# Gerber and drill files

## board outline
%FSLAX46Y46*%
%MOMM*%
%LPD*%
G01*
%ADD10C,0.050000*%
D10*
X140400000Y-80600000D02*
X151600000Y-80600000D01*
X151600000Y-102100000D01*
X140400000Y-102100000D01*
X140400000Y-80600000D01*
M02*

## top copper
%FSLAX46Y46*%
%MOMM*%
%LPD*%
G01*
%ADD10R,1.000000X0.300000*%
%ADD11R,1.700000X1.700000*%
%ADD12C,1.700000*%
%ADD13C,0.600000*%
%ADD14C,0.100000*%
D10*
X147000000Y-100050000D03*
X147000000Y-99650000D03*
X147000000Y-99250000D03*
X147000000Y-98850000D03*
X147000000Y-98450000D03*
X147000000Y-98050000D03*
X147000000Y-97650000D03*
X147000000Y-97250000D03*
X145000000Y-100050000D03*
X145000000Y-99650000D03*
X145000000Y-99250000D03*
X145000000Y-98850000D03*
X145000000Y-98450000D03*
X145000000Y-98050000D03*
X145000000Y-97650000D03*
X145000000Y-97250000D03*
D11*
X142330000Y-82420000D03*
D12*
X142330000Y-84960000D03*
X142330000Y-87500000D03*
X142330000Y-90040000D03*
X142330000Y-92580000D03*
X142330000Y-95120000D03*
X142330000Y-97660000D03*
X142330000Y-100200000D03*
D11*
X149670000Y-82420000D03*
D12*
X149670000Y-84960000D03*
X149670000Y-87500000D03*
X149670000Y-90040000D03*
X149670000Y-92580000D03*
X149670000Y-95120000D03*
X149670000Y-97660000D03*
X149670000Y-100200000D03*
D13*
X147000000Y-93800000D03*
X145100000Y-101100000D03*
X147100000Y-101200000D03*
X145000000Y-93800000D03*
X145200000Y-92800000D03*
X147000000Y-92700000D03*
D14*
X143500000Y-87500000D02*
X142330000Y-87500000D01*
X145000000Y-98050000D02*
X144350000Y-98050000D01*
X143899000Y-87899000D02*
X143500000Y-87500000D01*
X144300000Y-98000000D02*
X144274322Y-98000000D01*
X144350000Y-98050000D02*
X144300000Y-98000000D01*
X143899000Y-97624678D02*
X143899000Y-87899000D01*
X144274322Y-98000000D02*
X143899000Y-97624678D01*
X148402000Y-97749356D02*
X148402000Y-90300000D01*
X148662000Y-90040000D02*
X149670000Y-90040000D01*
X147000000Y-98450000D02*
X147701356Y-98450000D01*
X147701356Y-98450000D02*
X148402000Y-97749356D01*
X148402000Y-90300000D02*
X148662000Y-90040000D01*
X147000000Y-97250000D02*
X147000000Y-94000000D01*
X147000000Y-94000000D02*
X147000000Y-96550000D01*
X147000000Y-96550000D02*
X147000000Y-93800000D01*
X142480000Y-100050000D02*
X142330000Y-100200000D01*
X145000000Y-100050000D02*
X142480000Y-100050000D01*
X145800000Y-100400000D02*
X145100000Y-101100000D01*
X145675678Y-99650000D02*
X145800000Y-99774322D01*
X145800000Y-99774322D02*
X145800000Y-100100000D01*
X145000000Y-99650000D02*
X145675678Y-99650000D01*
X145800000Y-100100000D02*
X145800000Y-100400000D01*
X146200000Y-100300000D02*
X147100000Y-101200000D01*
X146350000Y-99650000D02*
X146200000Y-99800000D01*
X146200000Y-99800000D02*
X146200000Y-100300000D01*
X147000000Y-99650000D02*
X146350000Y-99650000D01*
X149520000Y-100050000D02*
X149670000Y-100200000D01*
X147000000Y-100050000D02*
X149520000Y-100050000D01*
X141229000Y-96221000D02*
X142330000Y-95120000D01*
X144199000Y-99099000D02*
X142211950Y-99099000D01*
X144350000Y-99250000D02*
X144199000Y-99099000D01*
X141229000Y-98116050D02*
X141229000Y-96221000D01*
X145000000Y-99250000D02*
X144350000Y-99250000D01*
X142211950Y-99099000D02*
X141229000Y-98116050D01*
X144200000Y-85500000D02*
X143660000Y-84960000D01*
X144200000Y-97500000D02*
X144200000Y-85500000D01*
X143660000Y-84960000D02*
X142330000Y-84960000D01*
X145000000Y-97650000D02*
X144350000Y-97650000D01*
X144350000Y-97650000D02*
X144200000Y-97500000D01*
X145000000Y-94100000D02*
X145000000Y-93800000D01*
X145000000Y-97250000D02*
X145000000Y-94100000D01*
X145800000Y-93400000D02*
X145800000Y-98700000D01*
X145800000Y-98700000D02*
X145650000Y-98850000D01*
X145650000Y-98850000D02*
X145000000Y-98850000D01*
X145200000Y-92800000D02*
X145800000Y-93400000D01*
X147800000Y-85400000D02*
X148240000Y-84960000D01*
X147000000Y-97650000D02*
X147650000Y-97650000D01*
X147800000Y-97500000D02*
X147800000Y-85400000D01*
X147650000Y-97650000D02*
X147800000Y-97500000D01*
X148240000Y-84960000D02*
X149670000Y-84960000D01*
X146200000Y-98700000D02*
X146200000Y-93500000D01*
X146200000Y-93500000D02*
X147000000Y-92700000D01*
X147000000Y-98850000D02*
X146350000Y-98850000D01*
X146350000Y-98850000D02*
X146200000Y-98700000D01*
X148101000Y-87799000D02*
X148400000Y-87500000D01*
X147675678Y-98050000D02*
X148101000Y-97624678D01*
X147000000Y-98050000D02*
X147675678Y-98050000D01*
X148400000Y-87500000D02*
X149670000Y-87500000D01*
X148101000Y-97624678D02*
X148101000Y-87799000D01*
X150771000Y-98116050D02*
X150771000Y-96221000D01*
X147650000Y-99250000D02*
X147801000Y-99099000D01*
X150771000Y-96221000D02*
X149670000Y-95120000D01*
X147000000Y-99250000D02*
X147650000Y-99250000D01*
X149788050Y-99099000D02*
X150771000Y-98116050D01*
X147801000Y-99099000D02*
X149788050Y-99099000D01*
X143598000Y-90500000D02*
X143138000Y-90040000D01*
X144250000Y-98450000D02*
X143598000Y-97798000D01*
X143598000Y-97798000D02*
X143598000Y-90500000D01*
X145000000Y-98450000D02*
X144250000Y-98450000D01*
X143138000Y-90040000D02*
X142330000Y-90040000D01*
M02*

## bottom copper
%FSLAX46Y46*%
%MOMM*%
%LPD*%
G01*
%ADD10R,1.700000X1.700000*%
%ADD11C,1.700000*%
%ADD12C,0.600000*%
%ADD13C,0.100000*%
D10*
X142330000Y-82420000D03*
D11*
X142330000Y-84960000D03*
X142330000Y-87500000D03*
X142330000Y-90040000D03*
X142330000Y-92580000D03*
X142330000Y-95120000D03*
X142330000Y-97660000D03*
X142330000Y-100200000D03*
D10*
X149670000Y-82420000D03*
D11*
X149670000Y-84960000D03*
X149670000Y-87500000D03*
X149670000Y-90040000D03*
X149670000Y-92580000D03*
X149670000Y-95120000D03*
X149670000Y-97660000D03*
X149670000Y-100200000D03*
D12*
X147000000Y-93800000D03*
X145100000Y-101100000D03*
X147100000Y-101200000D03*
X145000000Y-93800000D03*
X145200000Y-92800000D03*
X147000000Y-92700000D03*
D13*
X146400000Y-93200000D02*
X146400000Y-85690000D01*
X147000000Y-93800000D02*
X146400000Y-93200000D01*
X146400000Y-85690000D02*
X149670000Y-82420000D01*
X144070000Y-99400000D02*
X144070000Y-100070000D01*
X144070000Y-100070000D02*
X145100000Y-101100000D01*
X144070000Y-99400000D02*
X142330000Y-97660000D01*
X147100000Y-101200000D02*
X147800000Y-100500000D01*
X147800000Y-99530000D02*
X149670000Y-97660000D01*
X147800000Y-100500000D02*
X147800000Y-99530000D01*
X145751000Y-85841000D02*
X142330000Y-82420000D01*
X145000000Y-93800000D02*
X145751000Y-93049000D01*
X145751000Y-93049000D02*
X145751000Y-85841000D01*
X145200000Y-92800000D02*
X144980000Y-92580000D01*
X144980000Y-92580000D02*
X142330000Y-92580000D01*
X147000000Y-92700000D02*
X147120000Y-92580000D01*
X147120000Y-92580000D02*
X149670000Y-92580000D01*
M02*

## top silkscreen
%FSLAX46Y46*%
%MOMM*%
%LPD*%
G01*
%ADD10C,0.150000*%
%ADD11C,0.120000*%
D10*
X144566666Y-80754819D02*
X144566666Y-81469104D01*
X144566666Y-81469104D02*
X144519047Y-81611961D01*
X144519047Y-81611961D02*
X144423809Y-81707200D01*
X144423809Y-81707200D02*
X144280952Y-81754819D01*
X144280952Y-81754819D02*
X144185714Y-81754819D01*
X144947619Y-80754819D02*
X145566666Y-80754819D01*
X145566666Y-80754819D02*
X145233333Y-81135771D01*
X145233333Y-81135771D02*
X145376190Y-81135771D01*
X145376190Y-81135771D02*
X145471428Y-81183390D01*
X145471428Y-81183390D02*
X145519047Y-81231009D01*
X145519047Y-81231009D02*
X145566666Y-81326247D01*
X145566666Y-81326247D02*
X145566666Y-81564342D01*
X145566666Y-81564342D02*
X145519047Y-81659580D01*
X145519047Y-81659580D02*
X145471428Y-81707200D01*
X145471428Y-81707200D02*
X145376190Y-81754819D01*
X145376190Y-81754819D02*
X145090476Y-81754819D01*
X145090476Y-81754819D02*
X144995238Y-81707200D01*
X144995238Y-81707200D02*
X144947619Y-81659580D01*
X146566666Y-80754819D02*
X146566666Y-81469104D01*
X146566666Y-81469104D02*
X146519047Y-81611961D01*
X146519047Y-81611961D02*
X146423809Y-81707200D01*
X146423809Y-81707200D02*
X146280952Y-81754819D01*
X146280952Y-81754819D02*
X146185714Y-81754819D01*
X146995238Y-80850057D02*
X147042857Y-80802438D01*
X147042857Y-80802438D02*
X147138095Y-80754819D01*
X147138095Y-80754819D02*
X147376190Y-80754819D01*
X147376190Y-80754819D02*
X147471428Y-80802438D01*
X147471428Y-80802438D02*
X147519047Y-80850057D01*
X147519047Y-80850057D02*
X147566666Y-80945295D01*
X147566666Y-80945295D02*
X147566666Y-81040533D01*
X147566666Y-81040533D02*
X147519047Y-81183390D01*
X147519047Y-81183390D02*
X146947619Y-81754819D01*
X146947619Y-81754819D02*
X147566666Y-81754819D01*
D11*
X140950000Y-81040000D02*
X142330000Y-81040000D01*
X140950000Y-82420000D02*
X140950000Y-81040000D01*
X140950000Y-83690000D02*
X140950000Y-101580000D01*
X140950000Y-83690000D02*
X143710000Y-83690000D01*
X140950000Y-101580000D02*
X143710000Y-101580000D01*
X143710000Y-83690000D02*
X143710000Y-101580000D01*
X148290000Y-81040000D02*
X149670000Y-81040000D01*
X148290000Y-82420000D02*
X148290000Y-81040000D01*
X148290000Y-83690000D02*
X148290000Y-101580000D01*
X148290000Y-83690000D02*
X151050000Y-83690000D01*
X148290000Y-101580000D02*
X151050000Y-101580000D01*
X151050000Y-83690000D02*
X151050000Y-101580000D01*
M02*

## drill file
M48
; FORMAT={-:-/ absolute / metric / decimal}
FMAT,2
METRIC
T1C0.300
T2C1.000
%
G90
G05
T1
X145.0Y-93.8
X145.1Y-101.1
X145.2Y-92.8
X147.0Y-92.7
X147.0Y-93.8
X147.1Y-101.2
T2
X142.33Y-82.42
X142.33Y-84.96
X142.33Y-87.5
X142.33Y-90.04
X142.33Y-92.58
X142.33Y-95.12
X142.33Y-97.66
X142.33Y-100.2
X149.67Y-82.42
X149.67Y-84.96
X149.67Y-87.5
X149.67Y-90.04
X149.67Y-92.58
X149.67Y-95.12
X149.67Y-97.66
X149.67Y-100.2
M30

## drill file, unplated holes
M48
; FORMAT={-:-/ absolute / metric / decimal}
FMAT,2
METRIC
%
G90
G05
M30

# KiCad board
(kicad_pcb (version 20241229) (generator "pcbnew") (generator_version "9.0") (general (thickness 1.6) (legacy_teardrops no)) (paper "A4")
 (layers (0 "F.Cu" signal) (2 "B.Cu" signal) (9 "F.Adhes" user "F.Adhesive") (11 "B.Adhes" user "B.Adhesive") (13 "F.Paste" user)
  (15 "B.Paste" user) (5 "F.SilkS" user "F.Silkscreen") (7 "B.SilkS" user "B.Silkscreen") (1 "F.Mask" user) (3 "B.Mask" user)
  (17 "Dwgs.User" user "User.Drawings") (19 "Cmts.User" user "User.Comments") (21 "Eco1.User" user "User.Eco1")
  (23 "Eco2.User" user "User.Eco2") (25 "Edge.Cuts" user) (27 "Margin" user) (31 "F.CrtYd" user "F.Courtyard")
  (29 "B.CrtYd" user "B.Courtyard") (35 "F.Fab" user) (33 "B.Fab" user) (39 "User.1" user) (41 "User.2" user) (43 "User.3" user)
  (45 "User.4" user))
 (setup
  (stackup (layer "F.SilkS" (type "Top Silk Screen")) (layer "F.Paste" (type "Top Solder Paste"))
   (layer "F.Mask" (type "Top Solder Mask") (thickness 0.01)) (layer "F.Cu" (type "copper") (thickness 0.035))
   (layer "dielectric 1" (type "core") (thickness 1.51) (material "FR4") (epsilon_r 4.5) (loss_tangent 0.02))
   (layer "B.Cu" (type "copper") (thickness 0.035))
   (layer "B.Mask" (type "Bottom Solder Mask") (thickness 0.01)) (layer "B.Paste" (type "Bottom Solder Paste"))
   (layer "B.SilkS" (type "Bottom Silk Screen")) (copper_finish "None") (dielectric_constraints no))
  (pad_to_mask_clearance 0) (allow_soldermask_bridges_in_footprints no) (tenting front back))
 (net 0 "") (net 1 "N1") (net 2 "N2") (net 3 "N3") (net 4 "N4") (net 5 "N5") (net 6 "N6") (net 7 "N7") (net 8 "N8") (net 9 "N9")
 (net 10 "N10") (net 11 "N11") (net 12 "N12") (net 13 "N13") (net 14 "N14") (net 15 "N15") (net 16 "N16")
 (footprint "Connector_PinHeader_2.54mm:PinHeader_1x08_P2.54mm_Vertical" (layer "F.Cu") (at 142.33 82.42)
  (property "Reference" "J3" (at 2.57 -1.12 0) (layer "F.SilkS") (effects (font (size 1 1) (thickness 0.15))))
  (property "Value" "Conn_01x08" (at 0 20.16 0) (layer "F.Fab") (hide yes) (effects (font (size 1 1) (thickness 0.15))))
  (fp_line (start -1.38 -1.38) (end 0 -1.38) (stroke (width 0.12) (type solid)) (layer "F.SilkS"))
  (fp_line (start -1.38 0) (end -1.38 -1.38) (stroke (width 0.12) (type solid)) (layer "F.SilkS"))
  (fp_line (start -1.38 1.27) (end -1.38 19.16) (stroke (width 0.12) (type solid)) (layer "F.SilkS"))
  (fp_line (start -1.38 1.27) (end 1.38 1.27) (stroke (width 0.12) (type solid)) (layer "F.SilkS"))
  (fp_line (start -1.38 19.16) (end 1.38 19.16) (stroke (width 0.12) (type solid)) (layer "F.SilkS"))
  (fp_line (start 1.38 1.27) (end 1.38 19.16) (stroke (width 0.12) (type solid)) (layer "F.SilkS"))
  (pad "1" thru_hole rect (at 0 0) (size 1.7 1.7) (drill 1) (layers "*.Cu" "*.Mask") (remove_unused_layers no) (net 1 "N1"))
  (pad "2" thru_hole circle (at 0 2.54) (size 1.7 1.7) (drill 1) (layers "*.Cu" "*.Mask") (remove_unused_layers no) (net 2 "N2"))
  (pad "3" thru_hole circle (at 0 5.08) (size 1.7 1.7) (drill 1) (layers "*.Cu" "*.Mask") (remove_unused_layers no) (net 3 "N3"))
  (pad "4" thru_hole circle (at 0 7.62) (size 1.7 1.7) (drill 1) (layers "*.Cu" "*.Mask") (remove_unused_layers no) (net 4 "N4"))
  (pad "5" thru_hole circle (at 0 10.16) (size 1.7 1.7) (drill 1) (layers "*.Cu" "*.Mask") (remove_unused_layers no) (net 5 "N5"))
  (pad "6" thru_hole circle (at 0 12.7) (size 1.7 1.7) (drill 1) (layers "*.Cu" "*.Mask") (remove_unused_layers no) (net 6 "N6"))
  (pad "7" thru_hole circle (at 0 15.24) (size 1.7 1.7) (drill 1) (layers "*.Cu" "*.Mask") (remove_unused_layers no) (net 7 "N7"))
  (pad "8" thru_hole circle (at 0 17.78) (size 1.7 1.7) (drill 1) (layers "*.Cu" "*.Mask") (remove_unused_layers no) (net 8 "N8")))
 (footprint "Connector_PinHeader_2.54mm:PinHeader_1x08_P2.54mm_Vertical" (layer "F.Cu") (at 149.67 82.42)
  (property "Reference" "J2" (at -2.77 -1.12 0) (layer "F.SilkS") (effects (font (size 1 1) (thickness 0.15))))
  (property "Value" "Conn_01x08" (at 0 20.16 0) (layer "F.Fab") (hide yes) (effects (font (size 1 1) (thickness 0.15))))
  (fp_line (start -1.38 -1.38) (end 0 -1.38) (stroke (width 0.12) (type solid)) (layer "F.SilkS"))
  (fp_line (start -1.38 0) (end -1.38 -1.38) (stroke (width 0.12) (type solid)) (layer "F.SilkS"))
  (fp_line (start -1.38 1.27) (end -1.38 19.16) (stroke (width 0.12) (type solid)) (layer "F.SilkS"))
  (fp_line (start -1.38 1.27) (end 1.38 1.27) (stroke (width 0.12) (type solid)) (layer "F.SilkS"))
  (fp_line (start -1.38 19.16) (end 1.38 19.16) (stroke (width 0.12) (type solid)) (layer "F.SilkS"))
  (fp_line (start 1.38 1.27) (end 1.38 19.16) (stroke (width 0.12) (type solid)) (layer "F.SilkS"))
  (pad "1" thru_hole rect (at 0 0) (size 1.7 1.7) (drill 1) (layers "*.Cu" "*.Mask") (remove_unused_layers no) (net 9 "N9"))
  (pad "2" thru_hole circle (at 0 2.54) (size 1.7 1.7) (drill 1) (layers "*.Cu" "*.Mask") (remove_unused_layers no) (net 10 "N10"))
  (pad "3" thru_hole circle (at 0 5.08) (size 1.7 1.7) (drill 1) (layers "*.Cu" "*.Mask") (remove_unused_layers no) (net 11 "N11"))
  (pad "4" thru_hole circle (at 0 7.62) (size 1.7 1.7) (drill 1) (layers "*.Cu" "*.Mask") (remove_unused_layers no) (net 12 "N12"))
  (pad "5" thru_hole circle (at 0 10.16) (size 1.7 1.7) (drill 1) (layers "*.Cu" "*.Mask") (remove_unused_layers no) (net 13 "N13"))
  (pad "6" thru_hole circle (at 0 12.7) (size 1.7 1.7) (drill 1) (layers "*.Cu" "*.Mask") (remove_unused_layers no) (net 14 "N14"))
  (pad "7" thru_hole circle (at 0 15.24) (size 1.7 1.7) (drill 1) (layers "*.Cu" "*.Mask") (remove_unused_layers no) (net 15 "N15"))
  (pad "8" thru_hole circle (at 0 17.78) (size 1.7 1.7) (drill 1) (layers "*.Cu" "*.Mask") (remove_unused_layers no) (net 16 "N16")))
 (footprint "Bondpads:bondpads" (layer "F.Cu") (at 146 100.65)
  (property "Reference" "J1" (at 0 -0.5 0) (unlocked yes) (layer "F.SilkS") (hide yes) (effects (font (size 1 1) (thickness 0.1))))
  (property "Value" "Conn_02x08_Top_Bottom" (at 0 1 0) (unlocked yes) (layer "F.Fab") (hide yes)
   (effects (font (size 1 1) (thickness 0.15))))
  (pad "1" smd rect (at -1 -3.4) (size 1 0.3) (layers "F.Cu" "F.Mask" "F.Paste") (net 1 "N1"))
  (pad "2" smd rect (at -1 -3) (size 1 0.3) (layers "F.Cu" "F.Mask" "F.Paste") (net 2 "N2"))
  (pad "3" smd rect (at -1 -2.6) (size 1 0.3) (layers "F.Cu" "F.Mask" "F.Paste") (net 3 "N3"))
  (pad "4" smd rect (at -1 -2.2) (size 1 0.3) (layers "F.Cu" "F.Mask" "F.Paste") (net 4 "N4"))
  (pad "5" smd rect (at -1 -1.8) (size 1 0.3) (layers "F.Cu" "F.Mask" "F.Paste") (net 5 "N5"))
  (pad "6" smd rect (at -1 -1.4) (size 1 0.3) (layers "F.Cu" "F.Mask" "F.Paste") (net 6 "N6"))
  (pad "7" smd rect (at -1 -1) (size 1 0.3) (layers "F.Cu" "F.Mask" "F.Paste") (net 7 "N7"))
  (pad "8" smd rect (at -1 -0.6) (size 1 0.3) (layers "F.Cu" "F.Mask" "F.Paste") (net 8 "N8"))
  (pad "9" smd rect (at 1 -3.4) (size 1 0.3) (layers "F.Cu" "F.Mask" "F.Paste") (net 9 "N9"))
  (pad "10" smd rect (at 1 -3) (size 1 0.3) (layers "F.Cu" "F.Mask" "F.Paste") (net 10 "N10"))
  (pad "11" smd rect (at 1 -2.6) (size 1 0.3) (layers "F.Cu" "F.Mask" "F.Paste") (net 11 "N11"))
  (pad "12" smd rect (at 1 -2.2) (size 1 0.3) (layers "F.Cu" "F.Mask" "F.Paste") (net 12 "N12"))
  (pad "13" smd rect (at 1 -1.8) (size 1 0.3) (layers "F.Cu" "F.Mask" "F.Paste") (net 13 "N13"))
  (pad "14" smd rect (at 1 -1.4) (size 1 0.3) (layers "F.Cu" "F.Mask" "F.Paste") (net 14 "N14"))
  (pad "15" smd rect (at 1 -1) (size 1 0.3) (layers "F.Cu" "F.Mask" "F.Paste") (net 15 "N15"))
  (pad "16" smd rect (at 1 -0.6) (size 1 0.3) (layers "F.Cu" "F.Mask" "F.Paste") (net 16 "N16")))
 (gr_rect (start 140.4 80.6) (end 151.6 102.1) (stroke (width 0.05) (type default)) (fill no) (layer "Edge.Cuts"))
 (segment (start 143.5 87.5) (end 142.33 87.5) (width 0.1) (layer "F.Cu") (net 3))
 (segment (start 145 98.05) (end 144.35 98.05) (width 0.1) (layer "F.Cu") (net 3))
 (segment (start 143.899 87.899) (end 143.5 87.5) (width 0.1) (layer "F.Cu") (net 3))
 (segment (start 144.3 98) (end 144.274322 98) (width 0.1) (layer "F.Cu") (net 3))
 (segment (start 144.35 98.05) (end 144.3 98) (width 0.1) (layer "F.Cu") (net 3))
 (segment (start 143.899 97.624678) (end 143.899 87.899) (width 0.1) (layer "F.Cu") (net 3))
 (segment (start 144.274322 98) (end 143.899 97.624678) (width 0.1) (layer "F.Cu") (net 3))
 (segment (start 148.402 97.749356) (end 148.402 90.3) (width 0.1) (layer "F.Cu") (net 12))
 (segment (start 148.662 90.04) (end 149.67 90.04) (width 0.1) (layer "F.Cu") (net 12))
 (segment (start 147 98.45) (end 147.701356 98.45) (width 0.1) (layer "F.Cu") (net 12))
 (segment (start 147.701356 98.45) (end 148.402 97.749356) (width 0.1) (layer "F.Cu") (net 12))
 (segment (start 148.402 90.3) (end 148.662 90.04) (width 0.1) (layer "F.Cu") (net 12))
 (segment (start 147 97.25) (end 147 94) (width 0.1) (layer "F.Cu") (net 9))
 (segment (start 147 94) (end 147 96.55) (width 0.1) (layer "F.Cu") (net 9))
 (segment (start 147 96.55) (end 147 93.8) (width 0.1) (layer "F.Cu") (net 9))
 (via (at 147 93.8) (size 0.6) (drill 0.3) (layers "F.Cu" "B.Cu") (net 9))
 (segment (start 146.4 93.2) (end 146.4 85.69) (width 0.1) (layer "B.Cu") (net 9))
 (segment (start 147 93.8) (end 146.4 93.2) (width 0.1) (layer "B.Cu") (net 9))
 (segment (start 146.4 85.69) (end 149.67 82.42) (width 0.1) (layer "B.Cu") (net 9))
 (segment (start 142.48 100.05) (end 142.33 100.2) (width 0.1) (layer "F.Cu") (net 8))
 (segment (start 145 100.05) (end 142.48 100.05) (width 0.1) (layer "F.Cu") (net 8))
 (segment (start 145.8 100.4) (end 145.1 101.1) (width 0.1) (layer "F.Cu") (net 7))
 (segment (start 145.675678 99.65) (end 145.8 99.774322) (width 0.1) (layer "F.Cu") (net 7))
 (segment (start 145.8 99.774322) (end 145.8 100.1) (width 0.1) (layer "F.Cu") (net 7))
 (segment (start 145 99.65) (end 145.675678 99.65) (width 0.1) (layer "F.Cu") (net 7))
 (segment (start 145.8 100.1) (end 145.8 100.4) (width 0.1) (layer "F.Cu") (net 7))
 (via (at 145.1 101.1) (size 0.6) (drill 0.3) (layers "F.Cu" "B.Cu") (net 7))
 (segment (start 144.07 99.4) (end 144.07 100.07) (width 0.1) (layer "B.Cu") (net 7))
 (segment (start 144.07 100.07) (end 145.1 101.1) (width 0.1) (layer "B.Cu") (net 7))
 (segment (start 144.07 99.4) (end 142.33 97.66) (width 0.1) (layer "B.Cu") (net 7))
 (segment (start 146.2 100.3) (end 147.1 101.2) (width 0.1) (layer "F.Cu") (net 15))
 (segment (start 146.35 99.65) (end 146.2 99.8) (width 0.1) (layer "F.Cu") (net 15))
 (segment (start 146.2 99.8) (end 146.2 100.3) (width 0.1) (layer "F.Cu") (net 15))
 (segment (start 147 99.65) (end 146.35 99.65) (width 0.1) (layer "F.Cu") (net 15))
 (via (at 147.1 101.2) (size 0.6) (drill 0.3) (layers "F.Cu" "B.Cu") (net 15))
 (segment (start 147.1 101.2) (end 147.8 100.5) (width 0.1) (layer "B.Cu") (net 15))
 (segment (start 147.8 99.53) (end 149.67 97.66) (width 0.1) (layer "B.Cu") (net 15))
 (segment (start 147.8 100.5) (end 147.8 99.53) (width 0.1) (layer "B.Cu") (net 15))
 (segment (start 149.52 100.05) (end 149.67 100.2) (width 0.1) (layer "F.Cu") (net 16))
 (segment (start 147 100.05) (end 149.52 100.05) (width 0.1) (layer "F.Cu") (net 16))
 (segment (start 141.229 96.221) (end 142.33 95.12) (width 0.1) (layer "F.Cu") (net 6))
 (segment (start 144.199 99.099) (end 142.21195 99.099) (width 0.1) (layer "F.Cu") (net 6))
 (segment (start 144.35 99.25) (end 144.199 99.099) (width 0.1) (layer "F.Cu") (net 6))
 (segment (start 141.229 98.11605) (end 141.229 96.221) (width 0.1) (layer "F.Cu") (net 6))
 (segment (start 145 99.25) (end 144.35 99.25) (width 0.1) (layer "F.Cu") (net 6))
 (segment (start 142.21195 99.099) (end 141.229 98.11605) (width 0.1) (layer "F.Cu") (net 6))
 (segment (start 144.2 85.5) (end 143.66 84.96) (width 0.1) (layer "F.Cu") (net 2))
 (segment (start 144.2 97.5) (end 144.2 85.5) (width 0.1) (layer "F.Cu") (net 2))
 (segment (start 143.66 84.96) (end 142.33 84.96) (width 0.1) (layer "F.Cu") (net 2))
 (segment (start 145 97.65) (end 144.35 97.65) (width 0.1) (layer "F.Cu") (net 2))
 (segment (start 144.35 97.65) (end 144.2 97.5) (width 0.1) (layer "F.Cu") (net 2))
 (segment (start 145 94.1) (end 145 93.8) (width 0.1) (layer "F.Cu") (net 1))
 (segment (start 145 97.25) (end 145 94.1) (width 0.1) (layer "F.Cu") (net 1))
 (via (at 145 93.8) (size 0.6) (drill 0.3) (layers "F.Cu" "B.Cu") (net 1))
 (segment (start 145.751 85.841) (end 142.33 82.42) (width 0.1) (layer "B.Cu") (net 1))
 (segment (start 145 93.8) (end 145.751 93.049) (width 0.1) (layer "B.Cu") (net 1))
 (segment (start 145.751 93.049) (end 145.751 85.841) (width 0.1) (layer "B.Cu") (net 1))
 (segment (start 145.8 93.4) (end 145.8 98.7) (width 0.1) (layer "F.Cu") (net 5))
 (segment (start 145.8 98.7) (end 145.65 98.85) (width 0.1) (layer "F.Cu") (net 5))
 (segment (start 145.65 98.85) (end 145 98.85) (width 0.1) (layer "F.Cu") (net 5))
 (segment (start 145.2 92.8) (end 145.8 93.4) (width 0.1) (layer "F.Cu") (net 5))
 (via (at 145.2 92.8) (size 0.6) (drill 0.3) (layers "F.Cu" "B.Cu") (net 5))
 (segment (start 145.2 92.8) (end 144.98 92.58) (width 0.1) (layer "B.Cu") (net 5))
 (segment (start 144.98 92.58) (end 142.33 92.58) (width 0.1) (layer "B.Cu") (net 5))
 (segment (start 147.8 85.4) (end 148.24 84.96) (width 0.1) (layer "F.Cu") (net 10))
 (segment (start 147 97.65) (end 147.65 97.65) (width 0.1) (layer "F.Cu") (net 10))
 (segment (start 147.8 97.5) (end 147.8 85.4) (width 0.1) (layer "F.Cu") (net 10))
 (segment (start 147.65 97.65) (end 147.8 97.5) (width 0.1) (layer "F.Cu") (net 10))
 (segment (start 148.24 84.96) (end 149.67 84.96) (width 0.1) (layer "F.Cu") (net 10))
 (segment (start 146.2 98.7) (end 146.2 93.5) (width 0.1) (layer "F.Cu") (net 13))
 (segment (start 146.2 93.5) (end 147 92.7) (width 0.1) (layer "F.Cu") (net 13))
 (segment (start 147 98.85) (end 146.35 98.85) (width 0.1) (layer "F.Cu") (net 13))
 (segment (start 146.35 98.85) (end 146.2 98.7) (width 0.1) (layer "F.Cu") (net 13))
 (via (at 147 92.7) (size 0.6) (drill 0.3) (layers "F.Cu" "B.Cu") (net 13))
 (segment (start 147 92.7) (end 147.12 92.58) (width 0.1) (layer "B.Cu") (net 13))
 (segment (start 147.12 92.58) (end 149.67 92.58) (width 0.1) (layer "B.Cu") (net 13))
 (segment (start 148.101 87.799) (end 148.4 87.5) (width 0.1) (layer "F.Cu") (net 11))
 (segment (start 147.675678 98.05) (end 148.101 97.624678) (width 0.1) (layer "F.Cu") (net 11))
 (segment (start 147 98.05) (end 147.675678 98.05) (width 0.1) (layer "F.Cu") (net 11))
 (segment (start 148.4 87.5) (end 149.67 87.5) (width 0.1) (layer "F.Cu") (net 11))
 (segment (start 148.101 97.624678) (end 148.101 87.799) (width 0.1) (layer "F.Cu") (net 11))
 (segment (start 150.771 98.11605) (end 150.771 96.221) (width 0.1) (layer "F.Cu") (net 14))
 (segment (start 147.65 99.25) (end 147.801 99.099) (width 0.1) (layer "F.Cu") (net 14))
 (segment (start 150.771 96.221) (end 149.67 95.12) (width 0.1) (layer "F.Cu") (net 14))
 (segment (start 147 99.25) (end 147.65 99.25) (width 0.1) (layer "F.Cu") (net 14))
 (segment (start 149.78805 99.099) (end 150.771 98.11605) (width 0.1) (layer "F.Cu") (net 14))
 (segment (start 147.801 99.099) (end 149.78805 99.099) (width 0.1) (layer "F.Cu") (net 14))
 (segment (start 143.598 90.5) (end 143.138 90.04) (width 0.1) (layer "F.Cu") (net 4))
 (segment (start 144.25 98.45) (end 143.598 97.798) (width 0.1) (layer "F.Cu") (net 4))
 (segment (start 143.598 97.798) (end 143.598 90.5) (width 0.1) (layer "F.Cu") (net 4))
 (segment (start 145 98.45) (end 144.25 98.45) (width 0.1) (layer "F.Cu") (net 4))
 (segment (start 143.138 90.04) (end 142.33 90.04) (width 0.1) (layer "F.Cu") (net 4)))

